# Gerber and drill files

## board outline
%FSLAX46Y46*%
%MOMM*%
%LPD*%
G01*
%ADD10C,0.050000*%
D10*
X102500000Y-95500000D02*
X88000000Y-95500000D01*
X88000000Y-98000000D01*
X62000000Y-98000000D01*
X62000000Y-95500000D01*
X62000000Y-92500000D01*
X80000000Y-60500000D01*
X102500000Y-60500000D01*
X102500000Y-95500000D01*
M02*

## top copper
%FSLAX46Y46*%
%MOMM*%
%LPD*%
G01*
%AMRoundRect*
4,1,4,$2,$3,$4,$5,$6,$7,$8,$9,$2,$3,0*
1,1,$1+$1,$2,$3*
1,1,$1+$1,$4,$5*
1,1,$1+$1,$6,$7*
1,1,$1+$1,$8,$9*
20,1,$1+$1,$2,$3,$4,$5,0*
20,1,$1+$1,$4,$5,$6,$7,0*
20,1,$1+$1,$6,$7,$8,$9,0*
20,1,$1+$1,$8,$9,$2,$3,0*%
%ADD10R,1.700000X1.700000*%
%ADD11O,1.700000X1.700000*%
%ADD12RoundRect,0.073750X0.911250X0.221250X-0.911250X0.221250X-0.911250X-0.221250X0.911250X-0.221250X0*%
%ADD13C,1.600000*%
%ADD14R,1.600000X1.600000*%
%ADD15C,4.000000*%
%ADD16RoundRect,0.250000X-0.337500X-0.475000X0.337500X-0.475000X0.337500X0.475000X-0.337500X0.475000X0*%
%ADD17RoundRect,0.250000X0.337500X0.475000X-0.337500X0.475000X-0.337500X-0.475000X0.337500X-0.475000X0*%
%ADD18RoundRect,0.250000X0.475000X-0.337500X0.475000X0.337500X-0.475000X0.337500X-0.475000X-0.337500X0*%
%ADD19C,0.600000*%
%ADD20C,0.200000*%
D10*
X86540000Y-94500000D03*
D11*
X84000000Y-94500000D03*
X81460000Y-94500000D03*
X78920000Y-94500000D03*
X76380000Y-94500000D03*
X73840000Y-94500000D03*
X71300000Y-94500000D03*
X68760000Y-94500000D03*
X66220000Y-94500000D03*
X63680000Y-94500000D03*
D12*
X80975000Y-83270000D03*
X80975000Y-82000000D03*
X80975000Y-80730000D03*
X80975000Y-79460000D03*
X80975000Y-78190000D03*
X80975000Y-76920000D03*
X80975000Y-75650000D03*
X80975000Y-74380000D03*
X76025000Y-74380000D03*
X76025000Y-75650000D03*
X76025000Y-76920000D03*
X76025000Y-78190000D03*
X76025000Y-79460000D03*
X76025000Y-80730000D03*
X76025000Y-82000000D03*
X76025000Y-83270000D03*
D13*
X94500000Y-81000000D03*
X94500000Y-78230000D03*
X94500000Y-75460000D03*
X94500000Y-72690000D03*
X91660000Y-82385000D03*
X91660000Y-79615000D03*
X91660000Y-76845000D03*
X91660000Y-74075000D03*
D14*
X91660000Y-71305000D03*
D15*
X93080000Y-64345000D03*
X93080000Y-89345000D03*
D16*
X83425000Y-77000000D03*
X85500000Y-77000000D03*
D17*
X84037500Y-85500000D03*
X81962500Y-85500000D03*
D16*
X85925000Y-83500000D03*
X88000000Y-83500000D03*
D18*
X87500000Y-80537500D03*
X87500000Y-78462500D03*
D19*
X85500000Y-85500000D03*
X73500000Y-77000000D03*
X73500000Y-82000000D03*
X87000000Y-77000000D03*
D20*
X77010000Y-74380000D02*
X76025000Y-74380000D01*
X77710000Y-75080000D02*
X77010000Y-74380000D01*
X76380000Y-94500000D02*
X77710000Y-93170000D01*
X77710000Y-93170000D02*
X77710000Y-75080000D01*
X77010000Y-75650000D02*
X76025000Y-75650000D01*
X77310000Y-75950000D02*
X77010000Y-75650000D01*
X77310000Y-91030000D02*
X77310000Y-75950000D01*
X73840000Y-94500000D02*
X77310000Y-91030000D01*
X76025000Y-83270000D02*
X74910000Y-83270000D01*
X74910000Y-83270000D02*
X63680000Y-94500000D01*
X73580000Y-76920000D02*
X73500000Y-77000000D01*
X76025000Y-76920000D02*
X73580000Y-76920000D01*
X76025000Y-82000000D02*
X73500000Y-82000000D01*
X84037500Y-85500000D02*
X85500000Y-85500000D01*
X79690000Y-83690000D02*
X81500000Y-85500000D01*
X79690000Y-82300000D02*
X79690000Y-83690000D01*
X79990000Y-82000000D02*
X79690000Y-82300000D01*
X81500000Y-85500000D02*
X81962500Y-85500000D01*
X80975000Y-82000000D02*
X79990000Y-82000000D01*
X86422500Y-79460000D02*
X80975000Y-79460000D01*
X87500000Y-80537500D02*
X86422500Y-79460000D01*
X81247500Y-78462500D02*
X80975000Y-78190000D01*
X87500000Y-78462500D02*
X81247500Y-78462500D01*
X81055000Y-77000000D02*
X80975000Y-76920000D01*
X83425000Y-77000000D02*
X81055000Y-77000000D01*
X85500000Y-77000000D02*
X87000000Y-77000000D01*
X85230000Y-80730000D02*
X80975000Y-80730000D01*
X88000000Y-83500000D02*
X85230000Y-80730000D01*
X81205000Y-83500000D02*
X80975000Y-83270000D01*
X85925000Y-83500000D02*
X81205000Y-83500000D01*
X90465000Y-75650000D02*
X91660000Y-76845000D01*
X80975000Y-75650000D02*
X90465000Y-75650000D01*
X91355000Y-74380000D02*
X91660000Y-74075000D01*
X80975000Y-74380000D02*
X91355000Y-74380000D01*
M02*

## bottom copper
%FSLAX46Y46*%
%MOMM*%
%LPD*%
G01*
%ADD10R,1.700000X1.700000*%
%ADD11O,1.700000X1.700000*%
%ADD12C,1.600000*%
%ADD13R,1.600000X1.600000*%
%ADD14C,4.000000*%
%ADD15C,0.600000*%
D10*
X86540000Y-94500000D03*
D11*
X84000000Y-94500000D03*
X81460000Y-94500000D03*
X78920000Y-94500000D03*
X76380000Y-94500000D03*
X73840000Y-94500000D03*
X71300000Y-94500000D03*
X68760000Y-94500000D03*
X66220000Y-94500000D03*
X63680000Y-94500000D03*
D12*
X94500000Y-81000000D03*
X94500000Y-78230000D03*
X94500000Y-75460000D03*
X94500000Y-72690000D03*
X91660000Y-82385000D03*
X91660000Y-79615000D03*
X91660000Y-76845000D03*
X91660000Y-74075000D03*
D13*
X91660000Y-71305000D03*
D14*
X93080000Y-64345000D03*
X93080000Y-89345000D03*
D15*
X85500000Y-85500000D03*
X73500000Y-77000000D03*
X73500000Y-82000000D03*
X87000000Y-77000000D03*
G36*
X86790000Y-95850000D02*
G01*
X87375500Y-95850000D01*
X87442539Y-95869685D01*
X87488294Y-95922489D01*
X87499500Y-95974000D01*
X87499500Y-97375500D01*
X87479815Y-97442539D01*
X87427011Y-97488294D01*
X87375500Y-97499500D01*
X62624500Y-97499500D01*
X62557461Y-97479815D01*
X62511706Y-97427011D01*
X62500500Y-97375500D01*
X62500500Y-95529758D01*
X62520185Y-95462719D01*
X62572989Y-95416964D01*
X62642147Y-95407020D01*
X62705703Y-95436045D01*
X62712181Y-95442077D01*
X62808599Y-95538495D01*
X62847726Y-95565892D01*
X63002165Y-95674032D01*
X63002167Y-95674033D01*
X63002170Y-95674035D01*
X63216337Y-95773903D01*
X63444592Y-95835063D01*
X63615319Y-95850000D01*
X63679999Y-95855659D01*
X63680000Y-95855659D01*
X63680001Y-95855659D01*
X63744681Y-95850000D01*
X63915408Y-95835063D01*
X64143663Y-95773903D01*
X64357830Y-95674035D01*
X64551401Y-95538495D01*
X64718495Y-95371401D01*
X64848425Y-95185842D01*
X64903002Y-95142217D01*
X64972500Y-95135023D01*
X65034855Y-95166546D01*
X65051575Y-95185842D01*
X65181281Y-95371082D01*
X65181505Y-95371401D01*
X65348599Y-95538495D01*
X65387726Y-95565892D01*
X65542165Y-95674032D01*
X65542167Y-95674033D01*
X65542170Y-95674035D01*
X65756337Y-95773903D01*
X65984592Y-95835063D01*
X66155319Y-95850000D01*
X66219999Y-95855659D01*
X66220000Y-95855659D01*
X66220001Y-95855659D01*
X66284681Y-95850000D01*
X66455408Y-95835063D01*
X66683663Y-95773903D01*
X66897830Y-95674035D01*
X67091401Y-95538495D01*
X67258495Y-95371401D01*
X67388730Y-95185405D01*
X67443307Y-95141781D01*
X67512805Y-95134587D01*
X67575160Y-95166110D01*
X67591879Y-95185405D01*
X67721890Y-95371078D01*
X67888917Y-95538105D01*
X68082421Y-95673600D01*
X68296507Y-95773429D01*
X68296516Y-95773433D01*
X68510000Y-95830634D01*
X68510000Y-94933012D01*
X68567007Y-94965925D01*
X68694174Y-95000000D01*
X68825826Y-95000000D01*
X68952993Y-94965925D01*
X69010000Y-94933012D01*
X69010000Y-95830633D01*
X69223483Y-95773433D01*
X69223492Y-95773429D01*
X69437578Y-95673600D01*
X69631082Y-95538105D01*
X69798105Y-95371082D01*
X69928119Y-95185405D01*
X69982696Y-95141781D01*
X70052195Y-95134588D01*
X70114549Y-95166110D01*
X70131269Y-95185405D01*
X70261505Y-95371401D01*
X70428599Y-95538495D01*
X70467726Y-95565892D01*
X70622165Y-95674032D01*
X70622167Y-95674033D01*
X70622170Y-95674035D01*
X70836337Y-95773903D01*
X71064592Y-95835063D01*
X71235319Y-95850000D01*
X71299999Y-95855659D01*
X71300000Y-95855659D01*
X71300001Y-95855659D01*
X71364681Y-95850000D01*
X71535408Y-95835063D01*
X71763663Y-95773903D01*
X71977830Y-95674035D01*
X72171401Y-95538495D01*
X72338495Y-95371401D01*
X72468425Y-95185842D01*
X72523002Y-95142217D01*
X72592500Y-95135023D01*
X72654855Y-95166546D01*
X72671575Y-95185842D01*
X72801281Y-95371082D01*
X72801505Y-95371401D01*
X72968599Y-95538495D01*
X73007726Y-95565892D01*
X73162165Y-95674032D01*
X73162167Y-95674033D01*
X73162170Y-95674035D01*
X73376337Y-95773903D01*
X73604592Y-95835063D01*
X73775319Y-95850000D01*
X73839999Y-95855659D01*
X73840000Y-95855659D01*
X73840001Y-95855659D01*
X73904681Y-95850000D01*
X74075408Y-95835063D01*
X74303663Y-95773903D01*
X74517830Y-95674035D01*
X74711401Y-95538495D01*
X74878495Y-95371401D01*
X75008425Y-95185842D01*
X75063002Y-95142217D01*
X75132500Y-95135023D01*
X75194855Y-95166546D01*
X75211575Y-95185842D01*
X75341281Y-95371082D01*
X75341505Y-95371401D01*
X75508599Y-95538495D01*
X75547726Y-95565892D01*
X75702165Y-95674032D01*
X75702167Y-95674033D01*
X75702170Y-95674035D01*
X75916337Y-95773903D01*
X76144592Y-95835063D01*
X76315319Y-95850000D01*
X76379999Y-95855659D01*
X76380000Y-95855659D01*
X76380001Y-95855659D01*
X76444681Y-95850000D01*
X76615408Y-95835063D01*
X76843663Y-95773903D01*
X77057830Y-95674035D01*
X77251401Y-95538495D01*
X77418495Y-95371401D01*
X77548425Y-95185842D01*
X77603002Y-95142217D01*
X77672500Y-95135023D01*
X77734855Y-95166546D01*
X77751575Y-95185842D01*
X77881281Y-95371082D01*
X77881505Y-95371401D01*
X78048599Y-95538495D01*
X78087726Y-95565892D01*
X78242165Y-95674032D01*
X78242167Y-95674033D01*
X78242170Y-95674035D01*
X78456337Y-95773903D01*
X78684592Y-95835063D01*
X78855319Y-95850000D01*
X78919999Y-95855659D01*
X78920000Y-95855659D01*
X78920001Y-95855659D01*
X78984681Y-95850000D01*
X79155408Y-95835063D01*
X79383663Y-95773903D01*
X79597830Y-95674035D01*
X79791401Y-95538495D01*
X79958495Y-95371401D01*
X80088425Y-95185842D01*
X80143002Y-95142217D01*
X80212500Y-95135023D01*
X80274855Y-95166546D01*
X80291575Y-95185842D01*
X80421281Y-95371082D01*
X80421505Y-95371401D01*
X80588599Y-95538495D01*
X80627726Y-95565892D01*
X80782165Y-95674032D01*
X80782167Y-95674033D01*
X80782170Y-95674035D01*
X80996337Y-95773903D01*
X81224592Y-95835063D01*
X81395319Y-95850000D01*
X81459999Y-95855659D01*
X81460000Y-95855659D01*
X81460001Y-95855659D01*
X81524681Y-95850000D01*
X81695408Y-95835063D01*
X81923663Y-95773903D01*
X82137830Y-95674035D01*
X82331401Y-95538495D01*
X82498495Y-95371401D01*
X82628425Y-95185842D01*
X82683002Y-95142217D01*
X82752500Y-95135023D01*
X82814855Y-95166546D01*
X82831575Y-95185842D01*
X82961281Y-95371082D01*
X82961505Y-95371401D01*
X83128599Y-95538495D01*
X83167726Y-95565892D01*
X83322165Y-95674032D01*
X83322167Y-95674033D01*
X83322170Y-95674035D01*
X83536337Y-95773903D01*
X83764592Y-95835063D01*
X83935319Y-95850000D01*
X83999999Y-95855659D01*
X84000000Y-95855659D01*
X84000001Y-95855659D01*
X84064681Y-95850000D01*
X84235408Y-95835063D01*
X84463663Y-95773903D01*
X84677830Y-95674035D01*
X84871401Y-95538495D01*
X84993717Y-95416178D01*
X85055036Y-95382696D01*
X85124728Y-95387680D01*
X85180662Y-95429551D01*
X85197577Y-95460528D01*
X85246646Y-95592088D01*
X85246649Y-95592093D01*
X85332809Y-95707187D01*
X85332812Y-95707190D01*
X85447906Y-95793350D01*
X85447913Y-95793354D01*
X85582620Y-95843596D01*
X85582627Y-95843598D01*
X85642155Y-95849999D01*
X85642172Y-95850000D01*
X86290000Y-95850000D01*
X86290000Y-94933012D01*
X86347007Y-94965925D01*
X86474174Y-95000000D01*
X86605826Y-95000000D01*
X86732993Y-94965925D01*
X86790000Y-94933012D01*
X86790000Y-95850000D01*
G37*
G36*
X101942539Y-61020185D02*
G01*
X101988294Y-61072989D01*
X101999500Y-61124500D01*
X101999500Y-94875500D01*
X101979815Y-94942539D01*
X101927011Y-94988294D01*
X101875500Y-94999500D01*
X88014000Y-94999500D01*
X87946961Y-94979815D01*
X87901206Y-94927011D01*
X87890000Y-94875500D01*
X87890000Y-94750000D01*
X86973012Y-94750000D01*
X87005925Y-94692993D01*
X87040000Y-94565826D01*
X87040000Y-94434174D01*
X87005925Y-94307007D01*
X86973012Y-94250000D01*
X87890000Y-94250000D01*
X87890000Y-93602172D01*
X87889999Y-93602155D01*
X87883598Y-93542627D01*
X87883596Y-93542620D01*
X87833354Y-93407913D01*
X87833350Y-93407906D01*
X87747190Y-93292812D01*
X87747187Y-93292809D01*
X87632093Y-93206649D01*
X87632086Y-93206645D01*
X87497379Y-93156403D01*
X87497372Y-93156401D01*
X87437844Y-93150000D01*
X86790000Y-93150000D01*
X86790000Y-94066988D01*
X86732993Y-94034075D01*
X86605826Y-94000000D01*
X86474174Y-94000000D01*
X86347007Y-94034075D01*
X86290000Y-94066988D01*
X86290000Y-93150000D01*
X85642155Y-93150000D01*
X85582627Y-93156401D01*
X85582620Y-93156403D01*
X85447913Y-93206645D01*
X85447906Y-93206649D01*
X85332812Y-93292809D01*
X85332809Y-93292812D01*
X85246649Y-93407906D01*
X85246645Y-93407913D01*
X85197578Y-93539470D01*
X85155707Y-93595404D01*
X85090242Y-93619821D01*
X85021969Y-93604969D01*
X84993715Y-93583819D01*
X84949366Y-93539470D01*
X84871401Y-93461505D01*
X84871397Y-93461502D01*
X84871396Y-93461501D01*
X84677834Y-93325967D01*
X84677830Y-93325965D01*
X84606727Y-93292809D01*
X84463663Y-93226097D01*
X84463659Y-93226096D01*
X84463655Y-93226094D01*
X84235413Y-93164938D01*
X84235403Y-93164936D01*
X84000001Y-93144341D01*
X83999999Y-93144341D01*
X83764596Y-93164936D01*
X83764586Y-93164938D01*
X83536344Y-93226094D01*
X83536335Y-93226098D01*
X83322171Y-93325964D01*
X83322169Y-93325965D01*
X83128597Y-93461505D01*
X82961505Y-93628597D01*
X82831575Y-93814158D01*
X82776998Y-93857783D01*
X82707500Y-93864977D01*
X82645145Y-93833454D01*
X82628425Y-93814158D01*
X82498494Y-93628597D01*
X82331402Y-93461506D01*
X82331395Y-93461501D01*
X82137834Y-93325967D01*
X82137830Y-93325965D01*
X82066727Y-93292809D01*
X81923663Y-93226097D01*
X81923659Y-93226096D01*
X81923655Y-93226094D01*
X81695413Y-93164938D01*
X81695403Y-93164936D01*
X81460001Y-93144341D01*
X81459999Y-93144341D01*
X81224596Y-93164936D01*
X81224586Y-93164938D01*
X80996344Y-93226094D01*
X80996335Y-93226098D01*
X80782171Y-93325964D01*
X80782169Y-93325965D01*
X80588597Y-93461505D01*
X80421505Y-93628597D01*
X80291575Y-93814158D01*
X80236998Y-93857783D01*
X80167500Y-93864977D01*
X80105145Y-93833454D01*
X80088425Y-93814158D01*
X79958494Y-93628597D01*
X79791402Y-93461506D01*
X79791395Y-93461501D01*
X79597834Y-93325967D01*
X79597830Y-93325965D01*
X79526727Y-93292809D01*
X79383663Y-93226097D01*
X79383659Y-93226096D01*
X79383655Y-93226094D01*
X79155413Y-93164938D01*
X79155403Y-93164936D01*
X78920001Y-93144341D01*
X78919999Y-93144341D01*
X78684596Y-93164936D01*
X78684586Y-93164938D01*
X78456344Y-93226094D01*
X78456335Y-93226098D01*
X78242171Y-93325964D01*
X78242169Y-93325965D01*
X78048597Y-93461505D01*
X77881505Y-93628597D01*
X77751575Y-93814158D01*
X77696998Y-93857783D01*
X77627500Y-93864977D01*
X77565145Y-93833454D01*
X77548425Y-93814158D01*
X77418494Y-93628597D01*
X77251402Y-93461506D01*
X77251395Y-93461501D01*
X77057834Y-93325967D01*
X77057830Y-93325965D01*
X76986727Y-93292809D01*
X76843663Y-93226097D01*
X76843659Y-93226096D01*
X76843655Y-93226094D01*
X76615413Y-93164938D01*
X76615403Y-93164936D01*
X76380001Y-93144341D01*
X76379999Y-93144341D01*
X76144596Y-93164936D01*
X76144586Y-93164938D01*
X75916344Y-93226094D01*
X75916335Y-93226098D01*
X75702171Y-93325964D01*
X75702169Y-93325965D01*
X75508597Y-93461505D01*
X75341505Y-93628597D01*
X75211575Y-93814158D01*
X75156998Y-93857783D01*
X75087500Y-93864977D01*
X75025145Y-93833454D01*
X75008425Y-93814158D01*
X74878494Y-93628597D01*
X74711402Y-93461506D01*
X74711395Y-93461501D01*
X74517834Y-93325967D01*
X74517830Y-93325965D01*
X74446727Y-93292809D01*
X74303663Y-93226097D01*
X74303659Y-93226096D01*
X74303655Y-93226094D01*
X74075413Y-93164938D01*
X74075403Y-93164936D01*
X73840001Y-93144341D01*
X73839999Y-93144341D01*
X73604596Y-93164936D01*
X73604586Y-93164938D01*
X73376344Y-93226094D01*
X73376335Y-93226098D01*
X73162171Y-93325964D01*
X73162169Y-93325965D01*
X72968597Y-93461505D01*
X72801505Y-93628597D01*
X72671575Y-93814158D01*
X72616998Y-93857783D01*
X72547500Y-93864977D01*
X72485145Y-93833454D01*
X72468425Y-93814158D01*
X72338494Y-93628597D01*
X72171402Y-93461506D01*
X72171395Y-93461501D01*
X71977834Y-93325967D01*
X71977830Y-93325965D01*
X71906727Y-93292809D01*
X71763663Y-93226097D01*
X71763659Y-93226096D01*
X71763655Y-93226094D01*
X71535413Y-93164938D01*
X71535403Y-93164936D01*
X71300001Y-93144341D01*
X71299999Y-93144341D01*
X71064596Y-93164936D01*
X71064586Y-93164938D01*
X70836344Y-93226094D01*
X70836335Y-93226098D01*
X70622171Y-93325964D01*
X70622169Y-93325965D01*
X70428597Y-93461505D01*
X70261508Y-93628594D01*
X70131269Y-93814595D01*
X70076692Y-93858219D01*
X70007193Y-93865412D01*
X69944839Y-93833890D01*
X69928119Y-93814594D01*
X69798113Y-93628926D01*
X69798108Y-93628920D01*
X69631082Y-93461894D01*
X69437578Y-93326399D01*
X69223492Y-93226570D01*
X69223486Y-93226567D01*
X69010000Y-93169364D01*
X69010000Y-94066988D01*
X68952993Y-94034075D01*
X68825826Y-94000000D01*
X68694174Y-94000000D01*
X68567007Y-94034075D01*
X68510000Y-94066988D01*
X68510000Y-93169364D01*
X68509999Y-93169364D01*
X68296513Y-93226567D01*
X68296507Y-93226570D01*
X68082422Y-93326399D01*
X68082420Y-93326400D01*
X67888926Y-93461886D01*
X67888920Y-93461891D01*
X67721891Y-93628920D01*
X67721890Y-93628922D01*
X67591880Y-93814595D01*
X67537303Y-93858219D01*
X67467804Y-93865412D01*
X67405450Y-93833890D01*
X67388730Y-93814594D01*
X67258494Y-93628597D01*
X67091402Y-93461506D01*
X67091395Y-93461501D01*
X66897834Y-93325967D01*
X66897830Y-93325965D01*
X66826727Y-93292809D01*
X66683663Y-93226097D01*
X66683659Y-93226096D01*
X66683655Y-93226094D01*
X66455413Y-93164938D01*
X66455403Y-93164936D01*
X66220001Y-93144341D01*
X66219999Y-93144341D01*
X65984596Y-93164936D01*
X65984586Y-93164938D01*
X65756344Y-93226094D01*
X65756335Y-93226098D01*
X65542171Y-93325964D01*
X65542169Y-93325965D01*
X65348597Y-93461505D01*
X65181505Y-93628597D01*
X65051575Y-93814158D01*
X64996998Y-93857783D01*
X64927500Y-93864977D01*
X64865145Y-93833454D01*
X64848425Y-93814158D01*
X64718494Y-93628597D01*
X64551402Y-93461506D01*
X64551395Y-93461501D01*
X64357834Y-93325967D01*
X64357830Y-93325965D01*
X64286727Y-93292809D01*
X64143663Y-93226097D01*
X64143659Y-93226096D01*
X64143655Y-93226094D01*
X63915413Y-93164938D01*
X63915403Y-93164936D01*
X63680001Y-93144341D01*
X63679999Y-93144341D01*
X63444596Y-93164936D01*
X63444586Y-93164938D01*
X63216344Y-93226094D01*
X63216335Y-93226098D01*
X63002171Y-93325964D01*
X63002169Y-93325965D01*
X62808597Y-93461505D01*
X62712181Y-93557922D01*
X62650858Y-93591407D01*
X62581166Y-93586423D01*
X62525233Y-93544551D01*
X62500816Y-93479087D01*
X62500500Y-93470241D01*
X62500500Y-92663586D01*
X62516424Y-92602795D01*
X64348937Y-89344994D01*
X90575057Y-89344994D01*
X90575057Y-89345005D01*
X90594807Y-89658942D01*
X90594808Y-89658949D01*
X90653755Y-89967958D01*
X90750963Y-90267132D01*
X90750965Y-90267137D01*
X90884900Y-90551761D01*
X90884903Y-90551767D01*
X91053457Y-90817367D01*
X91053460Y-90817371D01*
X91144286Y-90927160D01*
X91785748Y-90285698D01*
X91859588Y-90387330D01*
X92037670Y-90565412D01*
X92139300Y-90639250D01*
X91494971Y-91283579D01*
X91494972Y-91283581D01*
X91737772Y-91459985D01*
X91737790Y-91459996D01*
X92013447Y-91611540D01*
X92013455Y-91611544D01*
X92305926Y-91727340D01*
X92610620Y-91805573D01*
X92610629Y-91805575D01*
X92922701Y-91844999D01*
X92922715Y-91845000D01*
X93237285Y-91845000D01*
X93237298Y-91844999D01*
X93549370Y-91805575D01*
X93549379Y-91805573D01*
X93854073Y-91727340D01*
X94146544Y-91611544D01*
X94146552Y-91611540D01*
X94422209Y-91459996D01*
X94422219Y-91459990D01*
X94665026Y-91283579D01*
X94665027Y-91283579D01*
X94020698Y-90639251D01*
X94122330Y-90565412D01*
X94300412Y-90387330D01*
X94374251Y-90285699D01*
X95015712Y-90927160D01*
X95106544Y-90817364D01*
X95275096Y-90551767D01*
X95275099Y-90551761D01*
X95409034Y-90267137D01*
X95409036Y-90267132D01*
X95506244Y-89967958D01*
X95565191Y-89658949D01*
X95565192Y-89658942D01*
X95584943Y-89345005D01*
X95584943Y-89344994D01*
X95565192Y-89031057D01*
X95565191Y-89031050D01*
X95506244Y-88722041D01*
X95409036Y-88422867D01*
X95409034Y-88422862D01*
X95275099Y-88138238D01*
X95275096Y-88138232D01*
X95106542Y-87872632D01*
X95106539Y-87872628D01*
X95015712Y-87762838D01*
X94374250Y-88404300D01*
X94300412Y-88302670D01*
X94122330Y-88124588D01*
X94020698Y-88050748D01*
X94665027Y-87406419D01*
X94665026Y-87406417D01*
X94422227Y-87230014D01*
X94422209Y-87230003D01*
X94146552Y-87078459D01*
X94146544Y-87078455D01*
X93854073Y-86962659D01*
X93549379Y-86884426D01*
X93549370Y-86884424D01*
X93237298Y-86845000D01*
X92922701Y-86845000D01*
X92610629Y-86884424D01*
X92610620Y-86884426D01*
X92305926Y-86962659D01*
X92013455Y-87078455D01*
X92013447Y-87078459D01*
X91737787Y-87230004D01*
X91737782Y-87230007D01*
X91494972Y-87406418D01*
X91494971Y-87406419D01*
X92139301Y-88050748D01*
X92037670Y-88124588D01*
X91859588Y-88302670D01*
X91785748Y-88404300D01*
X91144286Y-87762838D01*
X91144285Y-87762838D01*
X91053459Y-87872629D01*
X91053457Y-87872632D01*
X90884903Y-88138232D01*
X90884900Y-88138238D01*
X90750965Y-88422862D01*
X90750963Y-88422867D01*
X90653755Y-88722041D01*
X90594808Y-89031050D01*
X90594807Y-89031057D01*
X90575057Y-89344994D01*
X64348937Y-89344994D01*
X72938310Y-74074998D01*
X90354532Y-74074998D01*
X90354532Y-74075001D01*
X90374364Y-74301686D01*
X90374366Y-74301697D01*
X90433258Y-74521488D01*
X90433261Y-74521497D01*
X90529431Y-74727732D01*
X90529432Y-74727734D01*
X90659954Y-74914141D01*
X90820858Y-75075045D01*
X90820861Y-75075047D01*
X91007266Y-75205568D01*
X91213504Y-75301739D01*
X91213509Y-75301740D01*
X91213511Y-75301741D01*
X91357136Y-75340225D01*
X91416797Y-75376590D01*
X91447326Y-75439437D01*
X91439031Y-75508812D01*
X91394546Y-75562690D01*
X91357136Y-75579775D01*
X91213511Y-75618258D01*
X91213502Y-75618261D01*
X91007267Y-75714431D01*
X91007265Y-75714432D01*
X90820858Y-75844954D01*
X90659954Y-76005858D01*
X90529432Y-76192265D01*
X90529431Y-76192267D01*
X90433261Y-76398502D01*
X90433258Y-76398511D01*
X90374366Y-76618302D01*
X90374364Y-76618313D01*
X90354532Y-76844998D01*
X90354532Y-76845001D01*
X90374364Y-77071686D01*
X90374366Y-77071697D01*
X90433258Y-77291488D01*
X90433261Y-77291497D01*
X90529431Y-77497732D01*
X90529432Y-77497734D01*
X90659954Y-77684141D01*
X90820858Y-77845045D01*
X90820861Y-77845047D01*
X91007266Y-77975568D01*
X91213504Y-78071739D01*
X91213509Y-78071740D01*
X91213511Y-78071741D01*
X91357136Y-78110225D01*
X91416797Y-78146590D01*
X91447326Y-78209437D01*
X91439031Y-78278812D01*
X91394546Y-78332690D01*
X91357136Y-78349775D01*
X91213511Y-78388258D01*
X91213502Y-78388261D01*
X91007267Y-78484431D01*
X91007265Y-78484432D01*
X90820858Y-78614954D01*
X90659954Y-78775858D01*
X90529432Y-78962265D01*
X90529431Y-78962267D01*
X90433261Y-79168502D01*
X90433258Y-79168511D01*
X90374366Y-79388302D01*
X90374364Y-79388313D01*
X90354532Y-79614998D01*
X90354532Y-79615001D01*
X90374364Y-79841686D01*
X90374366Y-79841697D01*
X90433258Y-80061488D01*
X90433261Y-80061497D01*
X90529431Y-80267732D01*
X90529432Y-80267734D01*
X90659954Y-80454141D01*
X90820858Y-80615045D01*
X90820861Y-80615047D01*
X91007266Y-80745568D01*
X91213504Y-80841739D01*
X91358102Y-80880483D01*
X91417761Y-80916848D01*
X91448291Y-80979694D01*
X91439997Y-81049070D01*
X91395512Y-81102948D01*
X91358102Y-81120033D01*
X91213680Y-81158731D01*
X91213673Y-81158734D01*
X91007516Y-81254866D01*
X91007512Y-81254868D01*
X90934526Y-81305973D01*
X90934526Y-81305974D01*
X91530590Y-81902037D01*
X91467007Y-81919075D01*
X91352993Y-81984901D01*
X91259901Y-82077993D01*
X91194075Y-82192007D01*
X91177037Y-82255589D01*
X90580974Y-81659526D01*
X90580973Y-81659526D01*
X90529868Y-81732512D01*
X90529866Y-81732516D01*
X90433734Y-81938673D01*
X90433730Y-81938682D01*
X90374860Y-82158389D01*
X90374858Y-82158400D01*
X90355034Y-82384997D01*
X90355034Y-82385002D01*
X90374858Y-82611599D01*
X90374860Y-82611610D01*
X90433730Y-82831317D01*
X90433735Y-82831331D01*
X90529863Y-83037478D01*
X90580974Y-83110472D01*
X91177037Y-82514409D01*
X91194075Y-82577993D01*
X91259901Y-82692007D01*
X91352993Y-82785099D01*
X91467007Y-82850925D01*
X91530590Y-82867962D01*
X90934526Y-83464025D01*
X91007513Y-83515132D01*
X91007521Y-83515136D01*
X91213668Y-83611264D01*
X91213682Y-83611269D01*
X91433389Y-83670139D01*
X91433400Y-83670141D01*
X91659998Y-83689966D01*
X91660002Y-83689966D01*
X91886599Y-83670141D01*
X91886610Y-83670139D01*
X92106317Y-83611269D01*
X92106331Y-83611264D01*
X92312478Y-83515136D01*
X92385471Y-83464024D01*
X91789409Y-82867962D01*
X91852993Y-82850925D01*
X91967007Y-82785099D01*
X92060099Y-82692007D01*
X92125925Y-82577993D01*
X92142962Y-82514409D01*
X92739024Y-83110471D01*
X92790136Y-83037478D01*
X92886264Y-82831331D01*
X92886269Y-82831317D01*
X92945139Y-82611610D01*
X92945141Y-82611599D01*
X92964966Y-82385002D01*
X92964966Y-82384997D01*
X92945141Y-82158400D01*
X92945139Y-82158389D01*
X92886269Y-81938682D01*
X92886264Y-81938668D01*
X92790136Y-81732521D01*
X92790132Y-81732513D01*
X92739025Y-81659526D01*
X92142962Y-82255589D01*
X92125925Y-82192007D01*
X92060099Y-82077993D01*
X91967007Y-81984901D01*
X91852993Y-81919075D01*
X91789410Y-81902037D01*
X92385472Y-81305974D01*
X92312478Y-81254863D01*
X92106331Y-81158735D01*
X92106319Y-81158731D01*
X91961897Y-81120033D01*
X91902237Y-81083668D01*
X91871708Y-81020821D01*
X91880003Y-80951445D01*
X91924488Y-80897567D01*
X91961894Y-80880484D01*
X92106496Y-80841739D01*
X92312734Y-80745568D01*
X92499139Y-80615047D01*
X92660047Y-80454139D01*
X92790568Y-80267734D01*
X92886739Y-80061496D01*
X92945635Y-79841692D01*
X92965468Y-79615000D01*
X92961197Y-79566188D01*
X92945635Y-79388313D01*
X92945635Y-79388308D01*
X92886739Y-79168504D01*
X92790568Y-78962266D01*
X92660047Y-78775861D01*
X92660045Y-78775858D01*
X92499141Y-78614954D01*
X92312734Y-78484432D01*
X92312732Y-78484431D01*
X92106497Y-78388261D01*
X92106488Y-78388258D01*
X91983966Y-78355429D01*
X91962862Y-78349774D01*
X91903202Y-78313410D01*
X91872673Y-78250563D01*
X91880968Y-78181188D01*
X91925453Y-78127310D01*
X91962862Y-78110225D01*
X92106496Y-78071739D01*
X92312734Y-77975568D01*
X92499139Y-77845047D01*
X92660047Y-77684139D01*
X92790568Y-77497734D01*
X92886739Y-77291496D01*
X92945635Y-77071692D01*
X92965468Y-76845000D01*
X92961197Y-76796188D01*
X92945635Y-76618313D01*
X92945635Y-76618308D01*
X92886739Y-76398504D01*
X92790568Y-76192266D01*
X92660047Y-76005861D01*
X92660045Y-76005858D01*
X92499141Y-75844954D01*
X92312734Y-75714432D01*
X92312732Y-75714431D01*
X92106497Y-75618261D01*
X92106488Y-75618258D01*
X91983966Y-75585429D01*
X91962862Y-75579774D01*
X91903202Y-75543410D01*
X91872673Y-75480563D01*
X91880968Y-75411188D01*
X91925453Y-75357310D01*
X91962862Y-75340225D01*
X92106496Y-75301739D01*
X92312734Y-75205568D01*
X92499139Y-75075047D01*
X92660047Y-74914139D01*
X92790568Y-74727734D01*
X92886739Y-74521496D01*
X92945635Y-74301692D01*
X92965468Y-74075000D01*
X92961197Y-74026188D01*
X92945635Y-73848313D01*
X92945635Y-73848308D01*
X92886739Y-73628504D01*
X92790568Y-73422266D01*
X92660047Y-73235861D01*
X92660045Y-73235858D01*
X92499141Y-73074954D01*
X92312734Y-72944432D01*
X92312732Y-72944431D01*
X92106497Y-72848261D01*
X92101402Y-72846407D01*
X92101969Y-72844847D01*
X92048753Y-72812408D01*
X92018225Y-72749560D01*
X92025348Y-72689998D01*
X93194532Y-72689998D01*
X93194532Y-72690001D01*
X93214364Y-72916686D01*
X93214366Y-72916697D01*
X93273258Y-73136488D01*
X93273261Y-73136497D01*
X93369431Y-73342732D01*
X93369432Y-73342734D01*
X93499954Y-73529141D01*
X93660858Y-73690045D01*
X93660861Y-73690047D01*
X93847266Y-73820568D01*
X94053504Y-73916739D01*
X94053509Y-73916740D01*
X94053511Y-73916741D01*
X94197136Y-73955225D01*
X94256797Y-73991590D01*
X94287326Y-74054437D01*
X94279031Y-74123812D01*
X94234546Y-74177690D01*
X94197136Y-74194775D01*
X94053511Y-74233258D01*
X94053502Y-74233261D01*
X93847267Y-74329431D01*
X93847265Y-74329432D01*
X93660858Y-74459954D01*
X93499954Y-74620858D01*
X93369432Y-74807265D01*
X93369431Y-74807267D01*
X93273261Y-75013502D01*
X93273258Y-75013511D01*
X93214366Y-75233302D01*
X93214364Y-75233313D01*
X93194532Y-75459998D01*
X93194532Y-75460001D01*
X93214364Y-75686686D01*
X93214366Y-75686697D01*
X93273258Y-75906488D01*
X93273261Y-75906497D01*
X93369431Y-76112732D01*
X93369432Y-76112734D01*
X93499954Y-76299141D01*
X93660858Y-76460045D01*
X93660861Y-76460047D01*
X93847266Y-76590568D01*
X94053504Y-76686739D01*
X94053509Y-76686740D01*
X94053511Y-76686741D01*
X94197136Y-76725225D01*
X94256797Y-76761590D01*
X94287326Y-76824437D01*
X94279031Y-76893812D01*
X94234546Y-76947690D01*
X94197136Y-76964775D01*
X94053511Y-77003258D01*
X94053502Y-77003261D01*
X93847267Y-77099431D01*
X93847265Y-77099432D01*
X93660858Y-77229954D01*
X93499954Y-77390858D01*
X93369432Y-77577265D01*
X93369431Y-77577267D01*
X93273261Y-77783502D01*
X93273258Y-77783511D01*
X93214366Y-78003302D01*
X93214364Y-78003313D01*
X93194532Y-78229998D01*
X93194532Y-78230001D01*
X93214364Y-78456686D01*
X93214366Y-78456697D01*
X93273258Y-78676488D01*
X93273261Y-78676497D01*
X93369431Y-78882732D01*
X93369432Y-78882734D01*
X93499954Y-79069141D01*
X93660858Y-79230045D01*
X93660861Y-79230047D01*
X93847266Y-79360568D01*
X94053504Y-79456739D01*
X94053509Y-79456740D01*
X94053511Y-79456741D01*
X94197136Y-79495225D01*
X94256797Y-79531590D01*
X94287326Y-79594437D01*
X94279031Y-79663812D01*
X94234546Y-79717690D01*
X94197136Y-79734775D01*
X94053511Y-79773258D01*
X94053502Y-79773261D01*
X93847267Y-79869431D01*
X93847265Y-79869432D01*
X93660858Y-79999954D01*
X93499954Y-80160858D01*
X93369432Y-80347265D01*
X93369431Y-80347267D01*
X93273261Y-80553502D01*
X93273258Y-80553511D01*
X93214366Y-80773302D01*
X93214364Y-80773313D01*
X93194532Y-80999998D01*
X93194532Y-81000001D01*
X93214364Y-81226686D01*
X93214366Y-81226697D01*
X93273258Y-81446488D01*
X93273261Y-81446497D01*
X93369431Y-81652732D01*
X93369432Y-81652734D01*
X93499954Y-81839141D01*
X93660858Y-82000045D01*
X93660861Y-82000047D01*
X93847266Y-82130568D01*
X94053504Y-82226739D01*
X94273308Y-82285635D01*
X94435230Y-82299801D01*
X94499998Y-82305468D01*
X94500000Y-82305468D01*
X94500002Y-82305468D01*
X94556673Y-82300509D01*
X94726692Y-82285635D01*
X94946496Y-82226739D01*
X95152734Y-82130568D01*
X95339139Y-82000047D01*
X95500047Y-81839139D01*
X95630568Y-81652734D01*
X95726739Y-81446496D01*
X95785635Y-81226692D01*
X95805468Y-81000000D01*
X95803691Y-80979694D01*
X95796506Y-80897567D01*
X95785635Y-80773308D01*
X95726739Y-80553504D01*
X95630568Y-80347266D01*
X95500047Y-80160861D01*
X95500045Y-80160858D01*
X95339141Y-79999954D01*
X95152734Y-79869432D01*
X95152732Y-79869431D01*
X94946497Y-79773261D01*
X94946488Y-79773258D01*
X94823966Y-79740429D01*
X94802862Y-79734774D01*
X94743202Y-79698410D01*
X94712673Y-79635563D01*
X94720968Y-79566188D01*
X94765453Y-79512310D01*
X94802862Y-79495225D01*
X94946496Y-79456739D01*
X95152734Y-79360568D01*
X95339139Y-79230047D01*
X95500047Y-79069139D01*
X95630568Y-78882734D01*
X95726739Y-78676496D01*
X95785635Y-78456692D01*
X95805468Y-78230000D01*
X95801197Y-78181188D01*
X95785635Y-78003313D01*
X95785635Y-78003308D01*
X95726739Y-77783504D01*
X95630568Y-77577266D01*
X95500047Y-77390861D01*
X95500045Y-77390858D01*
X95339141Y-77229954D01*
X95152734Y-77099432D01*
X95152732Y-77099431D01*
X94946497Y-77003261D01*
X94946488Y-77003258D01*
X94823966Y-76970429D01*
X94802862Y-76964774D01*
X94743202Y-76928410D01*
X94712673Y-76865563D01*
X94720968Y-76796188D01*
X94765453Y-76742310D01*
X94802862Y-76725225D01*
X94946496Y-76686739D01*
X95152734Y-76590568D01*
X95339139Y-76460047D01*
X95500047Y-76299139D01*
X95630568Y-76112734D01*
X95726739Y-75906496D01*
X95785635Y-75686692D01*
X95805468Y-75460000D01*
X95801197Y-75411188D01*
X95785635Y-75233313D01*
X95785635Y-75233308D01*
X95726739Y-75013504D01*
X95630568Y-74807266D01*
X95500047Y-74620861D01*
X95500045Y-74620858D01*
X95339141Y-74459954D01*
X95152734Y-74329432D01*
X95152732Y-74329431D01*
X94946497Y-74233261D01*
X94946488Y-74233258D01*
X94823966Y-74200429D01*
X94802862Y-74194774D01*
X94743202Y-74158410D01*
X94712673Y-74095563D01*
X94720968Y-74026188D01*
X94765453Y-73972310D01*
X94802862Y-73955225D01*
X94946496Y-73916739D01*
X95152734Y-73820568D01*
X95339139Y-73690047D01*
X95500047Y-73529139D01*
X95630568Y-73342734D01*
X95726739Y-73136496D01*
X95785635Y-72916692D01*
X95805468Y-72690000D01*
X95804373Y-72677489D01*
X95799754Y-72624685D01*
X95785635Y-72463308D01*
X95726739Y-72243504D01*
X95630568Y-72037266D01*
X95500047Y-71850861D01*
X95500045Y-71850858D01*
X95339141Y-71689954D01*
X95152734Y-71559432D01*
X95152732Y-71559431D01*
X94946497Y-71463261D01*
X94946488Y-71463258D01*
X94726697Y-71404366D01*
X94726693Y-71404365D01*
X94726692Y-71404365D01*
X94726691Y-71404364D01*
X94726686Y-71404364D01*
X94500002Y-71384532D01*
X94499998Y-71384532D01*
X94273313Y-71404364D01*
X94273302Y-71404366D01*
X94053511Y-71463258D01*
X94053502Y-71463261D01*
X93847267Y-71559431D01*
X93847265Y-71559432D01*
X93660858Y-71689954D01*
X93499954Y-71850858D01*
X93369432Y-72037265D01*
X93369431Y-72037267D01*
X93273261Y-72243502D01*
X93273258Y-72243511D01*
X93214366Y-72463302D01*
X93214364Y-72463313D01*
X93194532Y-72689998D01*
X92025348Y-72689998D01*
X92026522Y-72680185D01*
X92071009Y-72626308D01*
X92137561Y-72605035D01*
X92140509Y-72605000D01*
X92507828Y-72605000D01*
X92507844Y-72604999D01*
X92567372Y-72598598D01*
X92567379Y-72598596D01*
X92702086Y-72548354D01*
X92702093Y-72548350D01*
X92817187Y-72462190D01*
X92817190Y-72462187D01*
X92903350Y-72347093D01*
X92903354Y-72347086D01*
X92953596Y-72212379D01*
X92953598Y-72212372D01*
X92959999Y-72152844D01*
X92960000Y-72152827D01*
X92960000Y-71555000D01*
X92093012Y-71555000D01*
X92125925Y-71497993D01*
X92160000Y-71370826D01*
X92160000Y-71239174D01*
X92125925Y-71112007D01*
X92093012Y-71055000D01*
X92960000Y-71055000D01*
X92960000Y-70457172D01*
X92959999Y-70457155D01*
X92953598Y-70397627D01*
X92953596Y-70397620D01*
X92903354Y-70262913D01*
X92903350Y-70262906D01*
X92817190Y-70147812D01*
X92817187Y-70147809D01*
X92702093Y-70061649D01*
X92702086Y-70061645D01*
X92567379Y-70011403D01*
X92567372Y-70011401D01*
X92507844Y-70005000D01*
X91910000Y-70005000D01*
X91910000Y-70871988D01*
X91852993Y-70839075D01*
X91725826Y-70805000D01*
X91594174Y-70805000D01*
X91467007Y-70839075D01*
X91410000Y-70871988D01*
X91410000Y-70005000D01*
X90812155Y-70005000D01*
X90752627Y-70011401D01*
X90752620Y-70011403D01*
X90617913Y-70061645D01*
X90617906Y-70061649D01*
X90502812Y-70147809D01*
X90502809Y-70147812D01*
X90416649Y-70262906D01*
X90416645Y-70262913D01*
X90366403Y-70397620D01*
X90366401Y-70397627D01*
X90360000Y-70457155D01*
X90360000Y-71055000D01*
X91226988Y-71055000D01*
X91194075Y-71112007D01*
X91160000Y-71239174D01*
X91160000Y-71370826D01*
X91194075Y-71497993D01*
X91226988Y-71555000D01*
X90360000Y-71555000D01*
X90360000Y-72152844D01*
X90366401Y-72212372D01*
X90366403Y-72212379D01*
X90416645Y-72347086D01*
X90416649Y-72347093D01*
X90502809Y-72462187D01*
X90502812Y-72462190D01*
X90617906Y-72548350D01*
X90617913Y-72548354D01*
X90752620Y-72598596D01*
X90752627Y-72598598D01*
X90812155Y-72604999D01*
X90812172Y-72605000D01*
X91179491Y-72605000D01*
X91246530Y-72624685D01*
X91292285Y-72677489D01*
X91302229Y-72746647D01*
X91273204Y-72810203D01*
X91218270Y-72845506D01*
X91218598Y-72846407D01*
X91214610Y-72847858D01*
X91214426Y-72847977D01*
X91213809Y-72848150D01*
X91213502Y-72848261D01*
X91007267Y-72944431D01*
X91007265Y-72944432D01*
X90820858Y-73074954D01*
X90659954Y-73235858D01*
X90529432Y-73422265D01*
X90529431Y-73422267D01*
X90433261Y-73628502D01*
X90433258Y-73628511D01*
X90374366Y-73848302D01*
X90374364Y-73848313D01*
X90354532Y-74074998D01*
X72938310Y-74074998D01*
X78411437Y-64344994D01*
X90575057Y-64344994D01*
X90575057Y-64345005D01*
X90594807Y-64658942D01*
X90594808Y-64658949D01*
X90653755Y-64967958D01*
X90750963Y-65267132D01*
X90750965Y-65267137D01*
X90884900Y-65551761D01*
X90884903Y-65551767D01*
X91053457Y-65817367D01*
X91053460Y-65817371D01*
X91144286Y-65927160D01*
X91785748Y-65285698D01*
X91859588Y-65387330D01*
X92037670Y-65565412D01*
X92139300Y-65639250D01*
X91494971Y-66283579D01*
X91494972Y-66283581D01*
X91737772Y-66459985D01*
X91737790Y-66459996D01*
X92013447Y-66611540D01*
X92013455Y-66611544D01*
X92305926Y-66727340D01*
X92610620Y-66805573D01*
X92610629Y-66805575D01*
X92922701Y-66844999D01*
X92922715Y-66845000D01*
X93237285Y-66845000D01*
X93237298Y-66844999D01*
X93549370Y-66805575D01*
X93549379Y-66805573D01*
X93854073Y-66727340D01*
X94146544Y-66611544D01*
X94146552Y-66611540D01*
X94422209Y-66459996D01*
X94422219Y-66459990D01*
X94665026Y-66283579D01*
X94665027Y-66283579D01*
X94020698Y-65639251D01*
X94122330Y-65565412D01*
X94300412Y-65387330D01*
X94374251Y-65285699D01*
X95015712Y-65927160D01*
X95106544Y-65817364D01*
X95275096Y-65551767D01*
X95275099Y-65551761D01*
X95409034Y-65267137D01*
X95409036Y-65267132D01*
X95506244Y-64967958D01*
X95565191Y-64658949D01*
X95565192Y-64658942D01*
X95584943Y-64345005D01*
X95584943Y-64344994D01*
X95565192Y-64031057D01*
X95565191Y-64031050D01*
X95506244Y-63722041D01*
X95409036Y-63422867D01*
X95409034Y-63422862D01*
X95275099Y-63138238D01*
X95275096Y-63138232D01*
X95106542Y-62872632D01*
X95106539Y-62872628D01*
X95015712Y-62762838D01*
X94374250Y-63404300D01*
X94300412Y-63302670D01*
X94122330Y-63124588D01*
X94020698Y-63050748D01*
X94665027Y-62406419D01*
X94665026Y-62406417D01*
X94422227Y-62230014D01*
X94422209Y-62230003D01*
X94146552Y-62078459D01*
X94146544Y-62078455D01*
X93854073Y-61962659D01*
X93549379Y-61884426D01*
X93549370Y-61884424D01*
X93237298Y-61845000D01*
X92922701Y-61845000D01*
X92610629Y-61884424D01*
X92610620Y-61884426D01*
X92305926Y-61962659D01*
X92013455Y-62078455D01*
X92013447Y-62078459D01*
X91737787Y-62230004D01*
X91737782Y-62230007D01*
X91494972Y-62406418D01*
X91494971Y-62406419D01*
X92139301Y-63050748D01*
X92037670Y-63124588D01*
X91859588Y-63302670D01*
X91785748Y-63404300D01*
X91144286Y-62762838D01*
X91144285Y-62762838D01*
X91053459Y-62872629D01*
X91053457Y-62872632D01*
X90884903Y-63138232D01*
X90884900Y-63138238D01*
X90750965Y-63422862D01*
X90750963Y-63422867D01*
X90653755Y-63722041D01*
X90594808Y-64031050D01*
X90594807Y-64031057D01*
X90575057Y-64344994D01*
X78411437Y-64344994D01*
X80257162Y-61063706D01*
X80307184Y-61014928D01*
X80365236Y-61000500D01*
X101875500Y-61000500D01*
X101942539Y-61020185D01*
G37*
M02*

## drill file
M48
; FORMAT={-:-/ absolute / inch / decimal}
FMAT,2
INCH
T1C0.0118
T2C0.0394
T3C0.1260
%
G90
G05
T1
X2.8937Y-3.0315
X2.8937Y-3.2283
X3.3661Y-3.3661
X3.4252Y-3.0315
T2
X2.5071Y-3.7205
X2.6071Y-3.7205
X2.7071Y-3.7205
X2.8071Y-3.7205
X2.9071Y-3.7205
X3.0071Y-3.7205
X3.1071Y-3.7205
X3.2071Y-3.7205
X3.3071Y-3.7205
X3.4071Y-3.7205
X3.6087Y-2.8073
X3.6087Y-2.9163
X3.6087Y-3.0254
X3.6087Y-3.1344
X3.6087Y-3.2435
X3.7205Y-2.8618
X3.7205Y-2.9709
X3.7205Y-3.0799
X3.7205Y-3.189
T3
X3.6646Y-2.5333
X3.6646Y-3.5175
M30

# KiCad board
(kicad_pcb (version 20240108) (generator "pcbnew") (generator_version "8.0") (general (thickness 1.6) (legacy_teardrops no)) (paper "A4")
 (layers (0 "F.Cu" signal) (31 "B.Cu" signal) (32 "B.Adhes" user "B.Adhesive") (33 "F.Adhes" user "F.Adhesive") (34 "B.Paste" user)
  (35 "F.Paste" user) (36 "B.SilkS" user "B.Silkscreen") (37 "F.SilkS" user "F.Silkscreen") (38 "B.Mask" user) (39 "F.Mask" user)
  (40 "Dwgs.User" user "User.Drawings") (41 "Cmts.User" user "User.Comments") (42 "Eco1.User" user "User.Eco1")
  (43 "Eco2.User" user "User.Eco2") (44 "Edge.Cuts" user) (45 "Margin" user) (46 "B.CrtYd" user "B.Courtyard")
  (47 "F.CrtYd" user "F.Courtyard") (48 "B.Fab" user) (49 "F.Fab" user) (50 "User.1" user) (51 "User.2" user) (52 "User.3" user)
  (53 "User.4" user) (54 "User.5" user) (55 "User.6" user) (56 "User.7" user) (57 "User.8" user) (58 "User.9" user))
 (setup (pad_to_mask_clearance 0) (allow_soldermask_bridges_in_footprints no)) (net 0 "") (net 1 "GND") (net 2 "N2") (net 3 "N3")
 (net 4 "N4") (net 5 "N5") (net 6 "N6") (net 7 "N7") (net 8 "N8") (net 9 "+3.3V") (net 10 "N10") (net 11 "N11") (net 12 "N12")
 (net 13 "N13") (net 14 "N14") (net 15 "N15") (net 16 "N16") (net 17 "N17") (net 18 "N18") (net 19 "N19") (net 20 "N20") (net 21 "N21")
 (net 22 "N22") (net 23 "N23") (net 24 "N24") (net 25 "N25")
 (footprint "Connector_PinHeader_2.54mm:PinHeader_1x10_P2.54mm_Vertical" (layer "F.Cu") (at 86.54 94.5 -90)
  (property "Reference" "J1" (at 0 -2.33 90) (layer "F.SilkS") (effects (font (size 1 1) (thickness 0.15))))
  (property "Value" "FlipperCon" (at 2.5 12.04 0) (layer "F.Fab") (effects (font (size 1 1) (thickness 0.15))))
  (pad "1" thru_hole rect (at 0 0 270) (size 1.7 1.7) (drill 1) (layers "*.Cu" "*.Mask") (remove_unused_layers no) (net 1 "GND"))
  (pad "2" thru_hole oval (at 0 2.54 270) (size 1.7 1.7) (drill 1) (layers "*.Cu" "*.Mask") (remove_unused_layers no) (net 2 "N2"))
  (pad "3" thru_hole oval (at 0 5.08 270) (size 1.7 1.7) (drill 1) (layers "*.Cu" "*.Mask") (remove_unused_layers no) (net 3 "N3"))
  (pad "4" thru_hole oval (at 0 7.62 270) (size 1.7 1.7) (drill 1) (layers "*.Cu" "*.Mask") (remove_unused_layers no) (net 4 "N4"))
  (pad "5" thru_hole oval (at 0 10.16 270) (size 1.7 1.7) (drill 1) (layers "*.Cu" "*.Mask") (remove_unused_layers no) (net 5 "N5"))
  (pad "6" thru_hole oval (at 0 12.7 270) (size 1.7 1.7) (drill 1) (layers "*.Cu" "*.Mask") (remove_unused_layers no) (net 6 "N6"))
  (pad "7" thru_hole oval (at 0 15.24 270) (size 1.7 1.7) (drill 1) (layers "*.Cu" "*.Mask") (remove_unused_layers no) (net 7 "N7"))
  (pad "8" thru_hole oval (at 0 17.78 270) (size 1.7 1.7) (drill 1) (layers "*.Cu" "*.Mask") (remove_unused_layers no) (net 1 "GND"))
  (pad "9" thru_hole oval (at 0 20.32 270) (size 1.7 1.7) (drill 1) (layers "*.Cu" "*.Mask") (remove_unused_layers no) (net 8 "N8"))
  (pad "10" thru_hole oval (at 0 22.86 270) (size 1.7 1.7) (drill 1) (layers "*.Cu" "*.Mask") (remove_unused_layers no) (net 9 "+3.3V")))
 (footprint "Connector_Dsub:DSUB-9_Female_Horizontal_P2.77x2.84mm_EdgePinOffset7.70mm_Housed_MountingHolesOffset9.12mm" (layer "F.Cu")
  (at 91.66 71.305 90)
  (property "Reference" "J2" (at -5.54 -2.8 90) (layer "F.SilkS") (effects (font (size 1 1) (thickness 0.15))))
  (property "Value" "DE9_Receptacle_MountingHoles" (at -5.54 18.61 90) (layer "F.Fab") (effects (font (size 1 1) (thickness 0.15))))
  (pad "0" thru_hole circle (at -18.04 1.42 90) (size 4 4) (drill 3.2) (layers "*.Cu" "*.Mask") (remove_unused_layers no) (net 1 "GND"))
  (pad "0" thru_hole circle (at 6.96 1.42 90) (size 4 4) (drill 3.2) (layers "*.Cu" "*.Mask") (remove_unused_layers no) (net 1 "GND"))
  (pad "1" thru_hole rect (at 0 0 90) (size 1.6 1.6) (drill 1) (layers "*.Cu" "*.Mask") (remove_unused_layers no) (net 1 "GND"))
  (pad "2" thru_hole circle (at -2.77 0 90) (size 1.6 1.6) (drill 1) (layers "*.Cu" "*.Mask") (remove_unused_layers no) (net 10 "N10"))
  (pad "3" thru_hole circle (at -5.54 0 90) (size 1.6 1.6) (drill 1) (layers "*.Cu" "*.Mask") (remove_unused_layers no) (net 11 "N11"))
  (pad "4" thru_hole circle (at -8.31 0 90) (size 1.6 1.6) (drill 1) (layers "*.Cu" "*.Mask") (remove_unused_layers no) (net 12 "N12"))
  (pad "5" thru_hole circle (at -11.08 0 90) (size 1.6 1.6) (drill 1) (layers "*.Cu" "*.Mask") (remove_unused_layers no) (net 1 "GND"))
  (pad "6" thru_hole circle (at -1.385 2.84 90) (size 1.6 1.6) (drill 1) (layers "*.Cu" "*.Mask") (remove_unused_layers no) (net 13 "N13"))
  (pad "7" thru_hole circle (at -4.155 2.84 90) (size 1.6 1.6) (drill 1) (layers "*.Cu" "*.Mask") (remove_unused_layers no) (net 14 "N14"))
  (pad "8" thru_hole circle (at -6.925 2.84 90) (size 1.6 1.6) (drill 1) (layers "*.Cu" "*.Mask") (remove_unused_layers no) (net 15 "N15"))
  (pad "9" thru_hole circle (at -9.695 2.84 90) (size 1.6 1.6) (drill 1) (layers "*.Cu" "*.Mask") (remove_unused_layers no) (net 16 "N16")))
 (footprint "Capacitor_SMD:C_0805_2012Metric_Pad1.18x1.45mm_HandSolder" (layer "F.Cu") (at 87.5 79.5 90)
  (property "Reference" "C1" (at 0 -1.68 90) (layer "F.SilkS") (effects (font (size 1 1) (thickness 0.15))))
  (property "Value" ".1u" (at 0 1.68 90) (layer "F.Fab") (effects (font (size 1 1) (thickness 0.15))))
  (pad "1" smd roundrect (at -1.0375 0 90) (size 1.175 1.45) (layers "F.Cu" "F.Paste" "F.Mask") (roundrect_rratio 0.212766) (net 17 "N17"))
  (pad "2" smd roundrect (at 1.0375 0 90) (size 1.175 1.45) (layers "F.Cu" "F.Paste" "F.Mask") (roundrect_rratio 0.212766) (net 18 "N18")))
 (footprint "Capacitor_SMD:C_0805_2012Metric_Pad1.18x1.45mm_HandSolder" (layer "F.Cu") (at 84.4625 77)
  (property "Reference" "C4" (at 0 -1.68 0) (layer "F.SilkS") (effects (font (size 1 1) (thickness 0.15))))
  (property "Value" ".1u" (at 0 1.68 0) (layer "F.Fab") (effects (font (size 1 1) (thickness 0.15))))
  (pad "1" smd roundrect (at -1.0375 0) (size 1.175 1.45) (layers "F.Cu" "F.Paste" "F.Mask") (roundrect_rratio 0.212766) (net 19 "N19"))
  (pad "2" smd roundrect (at 1.0375 0) (size 1.175 1.45) (layers "F.Cu" "F.Paste" "F.Mask") (roundrect_rratio 0.212766) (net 1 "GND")))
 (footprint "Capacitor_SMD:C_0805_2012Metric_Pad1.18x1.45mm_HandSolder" (layer "F.Cu") (at 83 85.5 180)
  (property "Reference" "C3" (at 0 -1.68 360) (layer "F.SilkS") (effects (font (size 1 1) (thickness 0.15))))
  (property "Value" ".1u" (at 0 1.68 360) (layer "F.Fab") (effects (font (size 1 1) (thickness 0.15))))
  (pad "1" smd roundrect (at -1.0375 0 180) (size 1.175 1.45) (layers "F.Cu" "F.Paste" "F.Mask") (roundrect_rratio 0.212766) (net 1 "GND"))
  (pad "2" smd roundrect (at 1.0375 0 180) (size 1.175 1.45) (layers "F.Cu" "F.Paste" "F.Mask") (roundrect_rratio 0.212766) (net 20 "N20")))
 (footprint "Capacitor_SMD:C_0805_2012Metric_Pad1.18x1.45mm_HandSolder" (layer "F.Cu") (at 86.9625 83.5)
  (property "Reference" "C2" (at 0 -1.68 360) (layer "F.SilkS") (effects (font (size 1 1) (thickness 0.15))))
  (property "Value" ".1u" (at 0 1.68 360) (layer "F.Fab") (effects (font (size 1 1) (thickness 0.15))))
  (pad "1" smd roundrect (at -1.0375 0) (size 1.175 1.45) (layers "F.Cu" "F.Paste" "F.Mask") (roundrect_rratio 0.212766) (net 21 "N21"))
  (pad "2" smd roundrect (at 1.0375 0) (size 1.175 1.45) (layers "F.Cu" "F.Paste" "F.Mask") (roundrect_rratio 0.212766) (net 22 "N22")))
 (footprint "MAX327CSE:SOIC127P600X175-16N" (layer "F.Cu") (at 78.5 78.825 180)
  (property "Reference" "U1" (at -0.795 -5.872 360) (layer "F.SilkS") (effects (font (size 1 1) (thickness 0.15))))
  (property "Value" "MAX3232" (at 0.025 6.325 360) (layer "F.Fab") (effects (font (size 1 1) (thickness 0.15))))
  (pad "1" smd roundrect (at -2.475 -4.445 180) (size 1.97 0.59) (layers "F.Cu" "F.Paste" "F.Mask") (roundrect_rratio 0.125) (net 21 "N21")
   (solder_mask_margin 0.102))
  (pad "2" smd roundrect (at -2.475 -3.175 180) (size 1.97 0.59) (layers "F.Cu" "F.Paste" "F.Mask") (roundrect_rratio 0.125) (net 20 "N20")
   (solder_mask_margin 0.102))
  (pad "3" smd roundrect (at -2.475 -1.905 180) (size 1.97 0.59) (layers "F.Cu" "F.Paste" "F.Mask") (roundrect_rratio 0.125) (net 22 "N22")
   (solder_mask_margin 0.102))
  (pad "4" smd roundrect (at -2.475 -0.635 180) (size 1.97 0.59) (layers "F.Cu" "F.Paste" "F.Mask") (roundrect_rratio 0.125) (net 17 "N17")
   (solder_mask_margin 0.102))
  (pad "5" smd roundrect (at -2.475 0.635 180) (size 1.97 0.59) (layers "F.Cu" "F.Paste" "F.Mask") (roundrect_rratio 0.125) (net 18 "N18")
   (solder_mask_margin 0.102))
  (pad "6" smd roundrect (at -2.475 1.905 180) (size 1.97 0.59) (layers "F.Cu" "F.Paste" "F.Mask") (roundrect_rratio 0.125) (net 19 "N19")
   (solder_mask_margin 0.102))
  (pad "7" smd roundrect (at -2.475 3.175 180) (size 1.97 0.59) (layers "F.Cu" "F.Paste" "F.Mask") (roundrect_rratio 0.125) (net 11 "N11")
   (solder_mask_margin 0.102))
  (pad "8" smd roundrect (at -2.475 4.445 180) (size 1.97 0.59) (layers "F.Cu" "F.Paste" "F.Mask") (roundrect_rratio 0.125) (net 10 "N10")
   (solder_mask_margin 0.102))
  (pad "9" smd roundrect (at 2.475 4.445 180) (size 1.97 0.59) (layers "F.Cu" "F.Paste" "F.Mask") (roundrect_rratio 0.125) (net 5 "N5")
   (solder_mask_margin 0.102))
  (pad "10" smd roundrect (at 2.475 3.175 180) (size 1.97 0.59) (layers "F.Cu" "F.Paste" "F.Mask") (roundrect_rratio 0.125) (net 6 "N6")
   (solder_mask_margin 0.102))
  (pad "11" smd roundrect (at 2.475 1.905 180) (size 1.97 0.59) (layers "F.Cu" "F.Paste" "F.Mask") (roundrect_rratio 0.125) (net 1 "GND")
   (solder_mask_margin 0.102))
  (pad "12" smd roundrect (at 2.475 0.635 180) (size 1.97 0.59) (layers "F.Cu" "F.Paste" "F.Mask") (roundrect_rratio 0.125) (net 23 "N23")
   (solder_mask_margin 0.102))
  (pad "13" smd roundrect (at 2.475 -0.635 180) (size 1.97 0.59) (layers "F.Cu" "F.Paste" "F.Mask") (roundrect_rratio 0.125) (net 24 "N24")
   (solder_mask_margin 0.102))
  (pad "14" smd roundrect (at 2.475 -1.905 180) (size 1.97 0.59) (layers "F.Cu" "F.Paste" "F.Mask") (roundrect_rratio 0.125) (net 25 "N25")
   (solder_mask_margin 0.102))
  (pad "15" smd roundrect (at 2.475 -3.175 180) (size 1.97 0.59) (layers "F.Cu" "F.Paste" "F.Mask") (roundrect_rratio 0.125) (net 1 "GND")
   (solder_mask_margin 0.102))
  (pad "16" smd roundrect (at 2.475 -4.445 180) (size 1.97 0.59) (layers "F.Cu" "F.Paste" "F.Mask") (roundrect_rratio 0.125) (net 9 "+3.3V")
   (solder_mask_margin 0.102)))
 (gr_poly
  (pts (xy 88 98) (xy 88 95.5) (xy 102.5 95.5) (xy 102.5 60.5) (xy 80 60.5) (xy 62 92.5) (xy 62 95.5) (xy 62 98))
  (stroke (width 0.05) (type solid)) (fill none) (layer "Edge.Cuts"))
 (segment (start 76.025 83.27) (end 74.91 83.27) (width 0.2) (layer "F.Cu") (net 9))
 (segment (start 74.91 83.27) (end 63.68 94.5) (width 0.2) (layer "F.Cu") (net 9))
 (segment (start 76.025 76.92) (end 73.58 76.92) (width 0.2) (layer "F.Cu") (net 1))
 (segment (start 73.58 76.92) (end 73.5 77) (width 0.2) (layer "F.Cu") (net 1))
 (segment (start 84.0375 85.5) (end 85.5 85.5) (width 0.2) (layer "F.Cu") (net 1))
 (segment (start 85.5 77) (end 87 77) (width 0.2) (layer "F.Cu") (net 1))
 (segment (start 76.025 82) (end 73.5 82) (width 0.2) (layer "F.Cu") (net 1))
 (via (at 73.5 82) (size 0.6) (drill 0.3) (layers "F.Cu" "B.Cu") (free yes) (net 1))
 (via (at 87 77) (size 0.6) (drill 0.3) (layers "F.Cu" "B.Cu") (free yes) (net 1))
 (via (at 73.5 77) (size 0.6) (drill 0.3) (layers "F.Cu" "B.Cu") (free yes) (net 1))
 (via (at 85.5 85.5) (size 0.6) (drill 0.3) (layers "F.Cu" "B.Cu") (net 1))
 (segment (start 86.4225 79.46) (end 80.975 79.46) (width 0.2) (layer "F.Cu") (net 17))
 (segment (start 87.5 80.5375) (end 86.4225 79.46) (width 0.2) (layer "F.Cu") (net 17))
 (segment (start 81.2475 78.4625) (end 80.975 78.19) (width 0.2) (layer "F.Cu") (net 18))
 (segment (start 87.5 78.4625) (end 81.2475 78.4625) (width 0.2) (layer "F.Cu") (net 18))
 (segment (start 85.925 83.5) (end 81.205 83.5) (width 0.2) (layer "F.Cu") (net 21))
 (segment (start 81.205 83.5) (end 80.975 83.27) (width 0.2) (layer "F.Cu") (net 21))
 (segment (start 88 83.5) (end 85.23 80.73) (width 0.2) (layer "F.Cu") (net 22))
 (segment (start 85.23 80.73) (end 80.975 80.73) (width 0.2) (layer "F.Cu") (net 22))
 (segment (start 83.425 77) (end 81.055 77) (width 0.2) (layer "F.Cu") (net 19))
 (segment (start 81.055 77) (end 80.975 76.92) (width 0.2) (layer "F.Cu") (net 19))
 (segment (start 80.975 74.38) (end 91.355 74.38) (width 0.2) (layer "F.Cu") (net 10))
 (segment (start 91.355 74.38) (end 91.66 74.075) (width 0.2) (layer "F.Cu") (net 10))
 (segment (start 80.975 75.65) (end 90.465 75.65) (width 0.2) (layer "F.Cu") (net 11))
 (segment (start 90.465 75.65) (end 91.66 76.845) (width 0.2) (layer "F.Cu") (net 11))
 (segment (start 79.99 82) (end 79.69 82.3) (width 0.2) (layer "F.Cu") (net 20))
 (segment (start 81.5 85.5) (end 81.9625 85.5) (width 0.2) (layer "F.Cu") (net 20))
 (segment (start 80.975 82) (end 79.99 82) (width 0.2) (layer "F.Cu") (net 20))
 (segment (start 79.69 82.3) (end 79.69 83.69) (width 0.2) (layer "F.Cu") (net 20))
 (segment (start 79.69 83.69) (end 81.5 85.5) (width 0.2) (layer "F.Cu") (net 20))
 (segment (start 77.31 75.95) (end 77.01 75.65) (width 0.2) (layer "F.Cu") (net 6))
 (segment (start 77.01 75.65) (end 76.025 75.65) (width 0.2) (layer "F.Cu") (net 6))
 (segment (start 73.84 94.5) (end 77.31 91.03) (width 0.2) (layer "F.Cu") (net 6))
 (segment (start 77.31 91.03) (end 77.31 75.95) (width 0.2) (layer "F.Cu") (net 6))
 (segment (start 76.38 94.5) (end 77.71 93.17) (width 0.2) (layer "F.Cu") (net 5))
 (segment (start 77.71 75.08) (end 77.01 74.38) (width 0.2) (layer "F.Cu") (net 5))
 (segment (start 77.71 93.17) (end 77.71 75.08) (width 0.2) (layer "F.Cu") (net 5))
 (segment (start 77.01 74.38) (end 76.025 74.38) (width 0.2) (layer "F.Cu") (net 5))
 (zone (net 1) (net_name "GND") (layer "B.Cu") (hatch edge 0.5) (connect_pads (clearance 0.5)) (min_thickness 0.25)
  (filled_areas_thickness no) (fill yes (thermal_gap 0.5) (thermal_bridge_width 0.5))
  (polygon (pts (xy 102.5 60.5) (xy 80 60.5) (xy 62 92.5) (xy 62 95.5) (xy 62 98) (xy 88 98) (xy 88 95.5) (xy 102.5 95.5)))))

